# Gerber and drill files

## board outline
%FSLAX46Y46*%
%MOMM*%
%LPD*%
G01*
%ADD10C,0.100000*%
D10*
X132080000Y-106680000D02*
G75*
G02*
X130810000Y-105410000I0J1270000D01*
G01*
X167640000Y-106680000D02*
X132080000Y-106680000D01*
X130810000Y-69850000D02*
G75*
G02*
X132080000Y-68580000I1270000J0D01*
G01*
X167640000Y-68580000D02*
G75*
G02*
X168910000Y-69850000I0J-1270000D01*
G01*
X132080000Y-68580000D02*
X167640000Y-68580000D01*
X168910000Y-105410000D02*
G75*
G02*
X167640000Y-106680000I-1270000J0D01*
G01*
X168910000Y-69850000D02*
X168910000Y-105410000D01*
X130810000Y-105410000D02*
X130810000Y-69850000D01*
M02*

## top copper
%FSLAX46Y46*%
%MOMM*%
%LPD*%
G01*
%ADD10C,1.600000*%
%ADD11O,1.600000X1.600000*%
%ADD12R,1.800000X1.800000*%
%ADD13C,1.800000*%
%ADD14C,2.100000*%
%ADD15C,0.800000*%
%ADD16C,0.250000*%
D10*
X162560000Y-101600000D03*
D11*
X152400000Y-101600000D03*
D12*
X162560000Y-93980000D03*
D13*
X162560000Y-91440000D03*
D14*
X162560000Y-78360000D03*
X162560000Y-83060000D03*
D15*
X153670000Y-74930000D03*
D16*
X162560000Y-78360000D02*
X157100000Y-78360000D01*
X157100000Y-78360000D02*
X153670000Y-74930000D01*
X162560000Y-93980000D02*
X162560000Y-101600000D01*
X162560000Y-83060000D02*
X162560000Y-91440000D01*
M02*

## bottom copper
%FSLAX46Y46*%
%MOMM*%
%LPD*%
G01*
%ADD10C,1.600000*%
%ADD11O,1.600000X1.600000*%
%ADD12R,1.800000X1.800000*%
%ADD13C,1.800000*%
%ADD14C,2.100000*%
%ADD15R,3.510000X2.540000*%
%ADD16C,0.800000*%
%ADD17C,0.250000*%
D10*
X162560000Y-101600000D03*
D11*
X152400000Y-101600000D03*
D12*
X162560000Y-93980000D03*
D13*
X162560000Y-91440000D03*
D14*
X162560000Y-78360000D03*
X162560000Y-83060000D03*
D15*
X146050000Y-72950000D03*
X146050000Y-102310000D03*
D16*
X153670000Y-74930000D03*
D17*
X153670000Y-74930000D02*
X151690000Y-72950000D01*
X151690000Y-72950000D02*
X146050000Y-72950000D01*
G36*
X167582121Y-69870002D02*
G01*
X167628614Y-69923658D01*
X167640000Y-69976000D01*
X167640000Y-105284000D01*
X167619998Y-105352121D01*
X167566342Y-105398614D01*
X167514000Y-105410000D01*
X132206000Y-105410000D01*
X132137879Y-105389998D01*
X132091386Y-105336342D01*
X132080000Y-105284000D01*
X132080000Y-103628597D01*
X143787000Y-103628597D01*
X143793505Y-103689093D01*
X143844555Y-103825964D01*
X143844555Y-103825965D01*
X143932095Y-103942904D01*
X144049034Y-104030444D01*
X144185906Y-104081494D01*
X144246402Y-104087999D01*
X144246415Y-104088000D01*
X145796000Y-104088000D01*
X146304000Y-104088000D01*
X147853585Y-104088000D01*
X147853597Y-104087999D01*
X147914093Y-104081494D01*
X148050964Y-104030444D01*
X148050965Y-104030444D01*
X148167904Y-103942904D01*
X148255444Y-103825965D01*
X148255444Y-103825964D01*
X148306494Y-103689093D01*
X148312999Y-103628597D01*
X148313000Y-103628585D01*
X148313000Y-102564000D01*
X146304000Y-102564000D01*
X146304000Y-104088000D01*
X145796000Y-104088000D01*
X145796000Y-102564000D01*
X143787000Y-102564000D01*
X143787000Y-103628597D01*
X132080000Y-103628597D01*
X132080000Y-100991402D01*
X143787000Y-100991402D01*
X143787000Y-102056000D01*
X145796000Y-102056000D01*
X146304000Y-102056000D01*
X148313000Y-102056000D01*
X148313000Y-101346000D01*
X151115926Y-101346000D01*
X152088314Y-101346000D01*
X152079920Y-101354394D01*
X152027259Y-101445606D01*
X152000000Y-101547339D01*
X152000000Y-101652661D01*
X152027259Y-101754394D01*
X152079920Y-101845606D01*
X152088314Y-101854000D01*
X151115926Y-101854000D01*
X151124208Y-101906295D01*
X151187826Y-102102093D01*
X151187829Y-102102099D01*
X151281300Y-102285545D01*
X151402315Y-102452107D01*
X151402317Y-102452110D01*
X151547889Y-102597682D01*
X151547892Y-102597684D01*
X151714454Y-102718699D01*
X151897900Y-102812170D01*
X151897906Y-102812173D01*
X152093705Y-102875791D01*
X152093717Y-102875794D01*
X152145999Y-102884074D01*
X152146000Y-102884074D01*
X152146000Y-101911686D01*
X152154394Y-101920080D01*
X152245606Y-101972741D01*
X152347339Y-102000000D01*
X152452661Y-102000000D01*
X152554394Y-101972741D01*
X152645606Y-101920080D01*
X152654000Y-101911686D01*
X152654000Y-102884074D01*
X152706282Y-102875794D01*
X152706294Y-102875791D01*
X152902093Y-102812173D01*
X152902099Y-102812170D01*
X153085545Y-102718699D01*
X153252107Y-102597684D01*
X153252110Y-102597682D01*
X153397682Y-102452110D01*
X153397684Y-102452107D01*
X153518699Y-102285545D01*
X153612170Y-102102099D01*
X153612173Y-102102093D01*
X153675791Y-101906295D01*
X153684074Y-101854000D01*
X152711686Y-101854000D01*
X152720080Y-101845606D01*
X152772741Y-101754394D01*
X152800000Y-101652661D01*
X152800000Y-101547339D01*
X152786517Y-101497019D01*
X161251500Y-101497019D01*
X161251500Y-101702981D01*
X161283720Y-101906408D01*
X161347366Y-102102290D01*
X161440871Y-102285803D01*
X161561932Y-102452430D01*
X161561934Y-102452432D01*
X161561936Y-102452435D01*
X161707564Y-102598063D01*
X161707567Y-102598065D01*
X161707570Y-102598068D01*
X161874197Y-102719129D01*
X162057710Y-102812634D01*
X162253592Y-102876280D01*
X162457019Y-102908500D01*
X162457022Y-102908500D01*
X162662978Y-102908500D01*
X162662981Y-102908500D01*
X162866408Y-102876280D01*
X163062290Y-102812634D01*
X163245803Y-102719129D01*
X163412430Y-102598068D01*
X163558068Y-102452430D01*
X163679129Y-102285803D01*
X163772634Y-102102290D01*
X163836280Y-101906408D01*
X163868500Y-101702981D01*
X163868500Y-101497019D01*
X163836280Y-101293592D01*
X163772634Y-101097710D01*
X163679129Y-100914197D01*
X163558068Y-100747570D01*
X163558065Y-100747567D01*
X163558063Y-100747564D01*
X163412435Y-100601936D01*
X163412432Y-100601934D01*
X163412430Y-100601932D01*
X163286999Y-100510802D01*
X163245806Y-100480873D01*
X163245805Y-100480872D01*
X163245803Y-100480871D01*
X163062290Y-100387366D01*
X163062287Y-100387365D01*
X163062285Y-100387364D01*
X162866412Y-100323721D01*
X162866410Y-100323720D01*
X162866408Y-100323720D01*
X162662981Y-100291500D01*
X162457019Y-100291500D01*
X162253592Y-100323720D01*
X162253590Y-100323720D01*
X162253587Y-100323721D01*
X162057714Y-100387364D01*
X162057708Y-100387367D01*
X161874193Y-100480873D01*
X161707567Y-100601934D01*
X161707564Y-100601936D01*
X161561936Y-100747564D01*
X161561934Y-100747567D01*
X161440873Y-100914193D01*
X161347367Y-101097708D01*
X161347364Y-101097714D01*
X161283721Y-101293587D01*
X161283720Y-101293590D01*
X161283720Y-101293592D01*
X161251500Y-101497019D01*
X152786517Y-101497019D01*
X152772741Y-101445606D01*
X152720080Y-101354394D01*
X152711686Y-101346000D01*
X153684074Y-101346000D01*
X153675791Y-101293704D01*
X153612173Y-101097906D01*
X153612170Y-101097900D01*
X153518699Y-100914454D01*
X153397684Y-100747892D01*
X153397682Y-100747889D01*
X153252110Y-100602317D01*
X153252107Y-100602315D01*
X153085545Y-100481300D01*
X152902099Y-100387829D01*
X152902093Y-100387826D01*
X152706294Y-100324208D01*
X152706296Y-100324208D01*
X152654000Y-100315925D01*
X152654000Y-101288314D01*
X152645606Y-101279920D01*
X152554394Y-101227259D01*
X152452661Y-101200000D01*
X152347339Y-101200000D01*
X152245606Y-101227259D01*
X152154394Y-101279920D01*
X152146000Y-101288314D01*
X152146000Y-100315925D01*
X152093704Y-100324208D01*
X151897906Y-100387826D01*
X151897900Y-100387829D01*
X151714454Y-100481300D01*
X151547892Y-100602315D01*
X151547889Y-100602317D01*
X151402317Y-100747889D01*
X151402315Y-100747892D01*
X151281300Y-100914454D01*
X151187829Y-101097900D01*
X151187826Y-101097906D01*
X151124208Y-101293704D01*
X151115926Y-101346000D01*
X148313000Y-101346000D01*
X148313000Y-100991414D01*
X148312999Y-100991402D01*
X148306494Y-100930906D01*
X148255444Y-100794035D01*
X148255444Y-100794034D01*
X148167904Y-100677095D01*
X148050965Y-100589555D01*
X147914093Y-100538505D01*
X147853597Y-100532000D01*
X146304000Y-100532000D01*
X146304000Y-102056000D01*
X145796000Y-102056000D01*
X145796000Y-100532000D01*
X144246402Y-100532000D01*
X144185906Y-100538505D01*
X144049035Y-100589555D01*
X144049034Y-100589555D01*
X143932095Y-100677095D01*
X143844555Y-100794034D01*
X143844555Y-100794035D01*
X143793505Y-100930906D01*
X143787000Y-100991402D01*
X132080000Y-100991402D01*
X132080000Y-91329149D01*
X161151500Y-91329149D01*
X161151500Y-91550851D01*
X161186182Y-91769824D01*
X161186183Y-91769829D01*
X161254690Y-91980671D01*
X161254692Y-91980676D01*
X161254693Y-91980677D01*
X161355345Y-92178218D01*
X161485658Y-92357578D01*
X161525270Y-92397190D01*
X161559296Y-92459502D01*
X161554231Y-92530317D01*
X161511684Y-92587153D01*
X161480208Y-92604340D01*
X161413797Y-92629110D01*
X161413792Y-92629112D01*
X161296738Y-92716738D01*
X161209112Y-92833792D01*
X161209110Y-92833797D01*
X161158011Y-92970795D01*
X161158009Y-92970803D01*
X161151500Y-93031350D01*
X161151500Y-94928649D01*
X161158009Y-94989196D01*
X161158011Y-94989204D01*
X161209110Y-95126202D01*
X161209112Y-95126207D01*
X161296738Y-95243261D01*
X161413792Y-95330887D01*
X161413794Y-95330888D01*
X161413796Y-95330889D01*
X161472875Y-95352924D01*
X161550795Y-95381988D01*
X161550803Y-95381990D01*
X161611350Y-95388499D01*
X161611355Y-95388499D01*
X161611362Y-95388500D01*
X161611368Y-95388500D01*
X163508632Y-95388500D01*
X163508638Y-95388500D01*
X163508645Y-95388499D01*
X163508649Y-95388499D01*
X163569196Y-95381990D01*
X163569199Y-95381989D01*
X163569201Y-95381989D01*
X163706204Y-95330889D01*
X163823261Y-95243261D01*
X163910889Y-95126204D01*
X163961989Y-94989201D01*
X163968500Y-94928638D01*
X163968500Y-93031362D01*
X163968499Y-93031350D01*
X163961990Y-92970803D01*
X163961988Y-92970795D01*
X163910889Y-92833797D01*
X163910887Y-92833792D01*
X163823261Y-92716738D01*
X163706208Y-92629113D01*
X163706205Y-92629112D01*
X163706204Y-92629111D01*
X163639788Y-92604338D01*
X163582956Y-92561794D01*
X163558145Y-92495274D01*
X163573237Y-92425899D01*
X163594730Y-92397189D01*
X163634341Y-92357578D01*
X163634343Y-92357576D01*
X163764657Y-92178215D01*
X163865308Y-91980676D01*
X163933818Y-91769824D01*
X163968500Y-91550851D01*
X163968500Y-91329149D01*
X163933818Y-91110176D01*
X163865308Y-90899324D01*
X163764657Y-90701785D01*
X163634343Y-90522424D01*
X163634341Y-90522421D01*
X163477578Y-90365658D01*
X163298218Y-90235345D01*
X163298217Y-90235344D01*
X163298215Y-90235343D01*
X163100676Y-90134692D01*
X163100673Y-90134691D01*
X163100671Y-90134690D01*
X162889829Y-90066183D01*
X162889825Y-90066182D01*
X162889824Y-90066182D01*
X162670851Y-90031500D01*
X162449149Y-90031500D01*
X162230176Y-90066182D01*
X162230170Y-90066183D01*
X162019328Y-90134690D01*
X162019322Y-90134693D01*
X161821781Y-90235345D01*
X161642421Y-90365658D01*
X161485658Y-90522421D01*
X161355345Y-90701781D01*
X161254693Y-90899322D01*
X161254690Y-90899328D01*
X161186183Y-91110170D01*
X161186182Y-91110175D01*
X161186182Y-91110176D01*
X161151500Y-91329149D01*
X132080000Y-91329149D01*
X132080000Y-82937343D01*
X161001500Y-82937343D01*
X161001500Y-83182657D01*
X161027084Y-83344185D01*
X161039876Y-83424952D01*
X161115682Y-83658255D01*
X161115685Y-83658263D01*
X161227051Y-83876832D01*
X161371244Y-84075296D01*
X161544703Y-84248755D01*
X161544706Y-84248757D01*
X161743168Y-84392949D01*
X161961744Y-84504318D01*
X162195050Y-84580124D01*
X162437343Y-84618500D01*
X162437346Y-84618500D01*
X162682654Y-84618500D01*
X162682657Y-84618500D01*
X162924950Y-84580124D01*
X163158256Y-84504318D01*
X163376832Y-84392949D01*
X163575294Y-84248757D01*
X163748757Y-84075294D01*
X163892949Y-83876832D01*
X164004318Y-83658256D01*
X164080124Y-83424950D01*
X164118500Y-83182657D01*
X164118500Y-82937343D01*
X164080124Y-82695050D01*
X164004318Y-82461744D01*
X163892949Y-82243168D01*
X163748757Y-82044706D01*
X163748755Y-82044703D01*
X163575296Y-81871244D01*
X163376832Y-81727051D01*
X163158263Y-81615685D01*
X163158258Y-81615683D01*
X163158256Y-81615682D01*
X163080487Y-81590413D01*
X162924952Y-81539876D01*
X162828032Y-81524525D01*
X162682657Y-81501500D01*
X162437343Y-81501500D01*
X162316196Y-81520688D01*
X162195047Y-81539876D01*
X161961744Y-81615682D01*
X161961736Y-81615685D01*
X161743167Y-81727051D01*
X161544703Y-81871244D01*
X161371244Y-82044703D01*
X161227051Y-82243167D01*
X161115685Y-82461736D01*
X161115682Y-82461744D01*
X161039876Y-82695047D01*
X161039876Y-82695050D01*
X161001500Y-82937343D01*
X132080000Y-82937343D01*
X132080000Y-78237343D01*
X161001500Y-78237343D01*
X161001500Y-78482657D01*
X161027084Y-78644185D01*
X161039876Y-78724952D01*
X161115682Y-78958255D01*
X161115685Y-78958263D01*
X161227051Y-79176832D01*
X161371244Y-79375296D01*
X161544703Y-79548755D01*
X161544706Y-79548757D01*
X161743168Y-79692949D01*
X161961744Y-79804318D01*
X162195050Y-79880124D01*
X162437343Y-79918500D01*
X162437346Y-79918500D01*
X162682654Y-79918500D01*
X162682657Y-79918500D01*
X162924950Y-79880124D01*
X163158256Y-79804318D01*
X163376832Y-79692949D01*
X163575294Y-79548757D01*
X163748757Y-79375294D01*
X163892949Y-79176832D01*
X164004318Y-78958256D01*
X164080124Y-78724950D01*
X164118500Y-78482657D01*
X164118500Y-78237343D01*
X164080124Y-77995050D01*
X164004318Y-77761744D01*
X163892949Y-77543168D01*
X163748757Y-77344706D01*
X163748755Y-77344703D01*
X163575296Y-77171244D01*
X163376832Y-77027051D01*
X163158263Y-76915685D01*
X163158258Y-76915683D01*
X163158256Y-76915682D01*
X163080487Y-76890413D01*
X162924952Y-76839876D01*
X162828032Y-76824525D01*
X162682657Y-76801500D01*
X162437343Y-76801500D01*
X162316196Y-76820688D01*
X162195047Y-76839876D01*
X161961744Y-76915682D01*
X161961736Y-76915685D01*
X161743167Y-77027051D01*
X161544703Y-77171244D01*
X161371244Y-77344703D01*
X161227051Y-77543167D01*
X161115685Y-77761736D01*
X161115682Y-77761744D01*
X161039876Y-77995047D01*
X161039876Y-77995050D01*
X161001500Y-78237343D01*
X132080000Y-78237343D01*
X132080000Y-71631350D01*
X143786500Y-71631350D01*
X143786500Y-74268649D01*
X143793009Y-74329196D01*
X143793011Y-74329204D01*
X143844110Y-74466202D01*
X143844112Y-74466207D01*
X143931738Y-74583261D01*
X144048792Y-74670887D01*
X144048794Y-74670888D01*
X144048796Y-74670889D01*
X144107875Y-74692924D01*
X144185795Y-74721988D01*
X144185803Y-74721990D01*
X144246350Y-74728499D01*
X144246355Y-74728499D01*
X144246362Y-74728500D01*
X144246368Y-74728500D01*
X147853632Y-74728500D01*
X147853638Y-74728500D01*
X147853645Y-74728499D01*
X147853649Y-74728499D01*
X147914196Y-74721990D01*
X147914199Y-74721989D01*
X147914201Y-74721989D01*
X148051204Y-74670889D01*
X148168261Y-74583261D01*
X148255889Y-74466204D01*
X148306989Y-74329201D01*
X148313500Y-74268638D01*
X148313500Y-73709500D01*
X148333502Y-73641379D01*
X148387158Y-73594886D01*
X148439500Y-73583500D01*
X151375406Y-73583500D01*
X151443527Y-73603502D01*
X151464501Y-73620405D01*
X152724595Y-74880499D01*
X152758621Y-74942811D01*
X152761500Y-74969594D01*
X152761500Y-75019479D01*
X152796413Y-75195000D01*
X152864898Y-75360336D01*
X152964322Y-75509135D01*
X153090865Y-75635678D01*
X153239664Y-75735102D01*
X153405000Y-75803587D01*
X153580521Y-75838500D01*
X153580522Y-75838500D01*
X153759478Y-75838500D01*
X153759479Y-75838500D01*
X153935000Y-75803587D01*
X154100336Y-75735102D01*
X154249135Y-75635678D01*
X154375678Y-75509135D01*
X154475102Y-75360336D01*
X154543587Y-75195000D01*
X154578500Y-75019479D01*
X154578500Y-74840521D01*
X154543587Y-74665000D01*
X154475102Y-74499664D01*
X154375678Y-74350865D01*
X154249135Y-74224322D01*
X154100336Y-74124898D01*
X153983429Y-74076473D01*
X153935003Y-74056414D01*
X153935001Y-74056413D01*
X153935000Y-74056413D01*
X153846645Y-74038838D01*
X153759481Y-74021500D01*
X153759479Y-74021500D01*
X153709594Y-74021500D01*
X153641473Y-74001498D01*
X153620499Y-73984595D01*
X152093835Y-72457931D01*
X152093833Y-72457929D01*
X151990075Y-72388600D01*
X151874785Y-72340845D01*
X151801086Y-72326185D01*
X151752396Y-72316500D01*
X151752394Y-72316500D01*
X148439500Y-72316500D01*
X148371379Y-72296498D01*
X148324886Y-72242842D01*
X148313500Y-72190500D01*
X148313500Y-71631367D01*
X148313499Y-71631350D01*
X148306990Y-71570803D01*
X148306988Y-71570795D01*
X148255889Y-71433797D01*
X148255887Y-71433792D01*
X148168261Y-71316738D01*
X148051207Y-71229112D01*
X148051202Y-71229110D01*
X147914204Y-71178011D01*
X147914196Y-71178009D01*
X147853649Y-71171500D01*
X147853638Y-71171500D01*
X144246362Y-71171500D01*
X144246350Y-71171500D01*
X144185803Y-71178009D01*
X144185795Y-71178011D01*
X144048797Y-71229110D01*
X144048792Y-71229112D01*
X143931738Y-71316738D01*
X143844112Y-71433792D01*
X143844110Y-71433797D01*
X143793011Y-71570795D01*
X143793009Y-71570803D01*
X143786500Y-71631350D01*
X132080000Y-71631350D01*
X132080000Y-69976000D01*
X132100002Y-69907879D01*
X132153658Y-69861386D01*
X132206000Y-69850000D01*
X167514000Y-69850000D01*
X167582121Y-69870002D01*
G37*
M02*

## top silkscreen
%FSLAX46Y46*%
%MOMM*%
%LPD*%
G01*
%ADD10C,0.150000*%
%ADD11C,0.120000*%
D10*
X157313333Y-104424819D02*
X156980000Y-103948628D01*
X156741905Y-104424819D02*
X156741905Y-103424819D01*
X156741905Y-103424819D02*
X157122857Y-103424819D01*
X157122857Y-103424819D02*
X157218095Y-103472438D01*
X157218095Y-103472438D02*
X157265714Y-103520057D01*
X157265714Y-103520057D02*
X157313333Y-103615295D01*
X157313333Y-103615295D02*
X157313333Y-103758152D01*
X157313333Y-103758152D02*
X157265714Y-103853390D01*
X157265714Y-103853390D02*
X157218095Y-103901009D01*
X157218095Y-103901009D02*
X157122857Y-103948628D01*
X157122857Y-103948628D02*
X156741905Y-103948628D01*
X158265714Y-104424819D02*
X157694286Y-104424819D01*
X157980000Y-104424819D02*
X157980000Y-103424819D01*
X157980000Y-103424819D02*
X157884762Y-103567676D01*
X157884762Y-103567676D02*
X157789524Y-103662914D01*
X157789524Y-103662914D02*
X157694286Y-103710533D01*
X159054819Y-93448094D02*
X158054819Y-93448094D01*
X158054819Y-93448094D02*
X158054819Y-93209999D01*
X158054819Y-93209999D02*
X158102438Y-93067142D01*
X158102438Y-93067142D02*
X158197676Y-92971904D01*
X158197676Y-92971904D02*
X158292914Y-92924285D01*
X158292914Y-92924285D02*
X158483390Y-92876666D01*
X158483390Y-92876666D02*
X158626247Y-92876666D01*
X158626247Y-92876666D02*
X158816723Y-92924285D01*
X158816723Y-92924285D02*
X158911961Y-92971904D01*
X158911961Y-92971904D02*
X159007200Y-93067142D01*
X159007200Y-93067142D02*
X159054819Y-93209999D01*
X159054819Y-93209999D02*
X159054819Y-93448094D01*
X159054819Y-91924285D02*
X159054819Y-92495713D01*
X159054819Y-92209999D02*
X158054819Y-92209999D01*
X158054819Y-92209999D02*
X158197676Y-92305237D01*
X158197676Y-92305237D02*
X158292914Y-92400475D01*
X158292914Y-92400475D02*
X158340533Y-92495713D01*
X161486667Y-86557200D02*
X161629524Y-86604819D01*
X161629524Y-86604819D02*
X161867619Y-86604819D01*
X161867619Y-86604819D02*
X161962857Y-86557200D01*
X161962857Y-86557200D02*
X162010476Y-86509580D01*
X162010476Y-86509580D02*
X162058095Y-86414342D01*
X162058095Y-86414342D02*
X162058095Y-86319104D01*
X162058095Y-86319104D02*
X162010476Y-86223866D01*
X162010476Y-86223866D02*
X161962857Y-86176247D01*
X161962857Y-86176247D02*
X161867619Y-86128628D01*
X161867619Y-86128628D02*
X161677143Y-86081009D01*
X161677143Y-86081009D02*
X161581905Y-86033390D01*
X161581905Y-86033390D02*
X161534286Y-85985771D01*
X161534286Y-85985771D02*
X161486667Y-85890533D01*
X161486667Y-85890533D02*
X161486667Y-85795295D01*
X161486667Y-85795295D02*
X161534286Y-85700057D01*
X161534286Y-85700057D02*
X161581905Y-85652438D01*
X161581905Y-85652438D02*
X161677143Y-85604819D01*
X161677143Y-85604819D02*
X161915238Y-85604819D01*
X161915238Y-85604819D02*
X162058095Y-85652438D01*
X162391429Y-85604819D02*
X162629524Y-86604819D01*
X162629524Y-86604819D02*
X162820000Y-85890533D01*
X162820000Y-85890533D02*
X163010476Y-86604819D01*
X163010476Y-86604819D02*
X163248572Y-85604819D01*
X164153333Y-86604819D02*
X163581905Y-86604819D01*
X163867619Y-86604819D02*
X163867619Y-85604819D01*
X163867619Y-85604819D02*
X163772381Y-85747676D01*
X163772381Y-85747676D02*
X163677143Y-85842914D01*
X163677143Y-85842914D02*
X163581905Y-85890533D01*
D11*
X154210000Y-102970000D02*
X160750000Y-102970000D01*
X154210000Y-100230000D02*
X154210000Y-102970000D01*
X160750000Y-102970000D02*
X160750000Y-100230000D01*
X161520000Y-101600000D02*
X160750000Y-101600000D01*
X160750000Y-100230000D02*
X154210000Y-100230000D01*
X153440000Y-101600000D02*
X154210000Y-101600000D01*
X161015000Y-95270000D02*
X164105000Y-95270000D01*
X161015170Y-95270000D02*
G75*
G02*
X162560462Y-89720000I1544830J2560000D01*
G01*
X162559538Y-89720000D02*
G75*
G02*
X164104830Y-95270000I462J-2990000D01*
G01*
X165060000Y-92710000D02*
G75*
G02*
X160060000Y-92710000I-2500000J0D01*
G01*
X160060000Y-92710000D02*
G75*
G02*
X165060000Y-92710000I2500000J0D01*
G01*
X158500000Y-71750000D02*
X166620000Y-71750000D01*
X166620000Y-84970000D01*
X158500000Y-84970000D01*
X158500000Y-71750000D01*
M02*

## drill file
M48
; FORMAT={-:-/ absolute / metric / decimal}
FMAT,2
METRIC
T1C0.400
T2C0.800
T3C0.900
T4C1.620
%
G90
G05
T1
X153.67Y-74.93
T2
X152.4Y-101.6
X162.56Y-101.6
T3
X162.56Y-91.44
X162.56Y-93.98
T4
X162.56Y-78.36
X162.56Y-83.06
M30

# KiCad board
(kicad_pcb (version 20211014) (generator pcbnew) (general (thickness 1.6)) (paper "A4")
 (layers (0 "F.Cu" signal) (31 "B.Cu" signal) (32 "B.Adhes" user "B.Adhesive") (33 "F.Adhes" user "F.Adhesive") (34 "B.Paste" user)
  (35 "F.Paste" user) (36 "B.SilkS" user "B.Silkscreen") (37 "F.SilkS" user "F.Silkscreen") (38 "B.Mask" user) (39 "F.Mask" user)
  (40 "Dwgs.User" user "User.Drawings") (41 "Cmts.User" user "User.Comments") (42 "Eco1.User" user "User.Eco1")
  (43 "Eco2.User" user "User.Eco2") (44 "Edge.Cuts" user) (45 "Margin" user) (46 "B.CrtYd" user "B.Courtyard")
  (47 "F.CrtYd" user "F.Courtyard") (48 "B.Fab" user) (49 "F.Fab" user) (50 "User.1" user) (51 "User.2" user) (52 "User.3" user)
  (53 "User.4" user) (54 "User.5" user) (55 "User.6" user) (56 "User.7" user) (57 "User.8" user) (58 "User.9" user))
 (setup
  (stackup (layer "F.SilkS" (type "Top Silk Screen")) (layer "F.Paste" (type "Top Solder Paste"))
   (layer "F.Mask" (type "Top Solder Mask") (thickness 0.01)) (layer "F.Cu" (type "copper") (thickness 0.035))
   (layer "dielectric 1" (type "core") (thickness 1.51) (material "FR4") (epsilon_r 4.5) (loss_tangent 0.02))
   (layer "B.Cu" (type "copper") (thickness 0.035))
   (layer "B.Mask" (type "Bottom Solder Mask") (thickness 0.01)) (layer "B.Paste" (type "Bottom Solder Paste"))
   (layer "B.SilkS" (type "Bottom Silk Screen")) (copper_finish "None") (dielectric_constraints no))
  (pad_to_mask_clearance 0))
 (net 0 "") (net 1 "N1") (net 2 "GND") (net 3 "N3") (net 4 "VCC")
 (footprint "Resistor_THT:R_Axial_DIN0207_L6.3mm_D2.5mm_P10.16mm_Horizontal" (layer "F.Cu") (at 162.56 101.6 180)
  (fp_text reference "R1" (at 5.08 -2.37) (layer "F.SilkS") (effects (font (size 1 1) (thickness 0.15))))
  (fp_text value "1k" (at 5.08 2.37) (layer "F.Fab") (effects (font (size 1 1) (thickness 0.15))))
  (fp_line (start 8.35 -1.37) (end 1.81 -1.37) (layer "F.SilkS") (width 0.12))
  (fp_line (start 8.35 1.37) (end 8.35 -1.37) (layer "F.SilkS") (width 0.12))
  (fp_line (start 1.81 -1.37) (end 1.81 1.37) (layer "F.SilkS") (width 0.12))
  (fp_line (start 1.04 0) (end 1.81 0) (layer "F.SilkS") (width 0.12))
  (fp_line (start 1.81 1.37) (end 8.35 1.37) (layer "F.SilkS") (width 0.12))
  (fp_line (start 9.12 0) (end 8.35 0) (layer "F.SilkS") (width 0.12))
  (pad "1" thru_hole circle (at 0 0 180) (size 1.6 1.6) (drill 0.8) (layers *.Cu *.Mask) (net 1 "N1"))
  (pad "2" thru_hole oval (at 10.16 0 180) (size 1.6 1.6) (drill 0.8) (layers *.Cu *.Mask) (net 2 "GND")))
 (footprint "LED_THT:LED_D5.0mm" (layer "F.Cu") (at 162.56 93.98 90)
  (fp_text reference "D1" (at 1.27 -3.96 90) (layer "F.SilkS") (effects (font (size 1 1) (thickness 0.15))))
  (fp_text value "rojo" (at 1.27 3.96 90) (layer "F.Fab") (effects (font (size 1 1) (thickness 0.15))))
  (fp_line (start -1.29 -1.545) (end -1.29 1.545) (layer "F.SilkS") (width 0.12))
  (fp_arc (start -1.29 -1.54483) (mid 2.072002 -2.880433) (end 4.26 0.000462) (layer "F.SilkS") (width 0.12))
  (fp_arc (start 4.26 -0.000462) (mid 2.072002 2.880433) (end -1.29 1.54483) (layer "F.SilkS") (width 0.12))
  (fp_circle (center 1.27 0) (end 3.77 0) (layer "F.SilkS") (width 0.12) (fill none))
  (pad "1" thru_hole rect (at 0 0 90) (size 1.8 1.8) (drill 0.9) (layers *.Cu *.Mask) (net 1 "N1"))
  (pad "2" thru_hole circle (at 2.54 0 90) (size 1.8 1.8) (drill 0.9) (layers *.Cu *.Mask) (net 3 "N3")))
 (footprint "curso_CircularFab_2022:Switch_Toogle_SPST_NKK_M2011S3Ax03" (layer "F.Cu") (at 162.56 73.66)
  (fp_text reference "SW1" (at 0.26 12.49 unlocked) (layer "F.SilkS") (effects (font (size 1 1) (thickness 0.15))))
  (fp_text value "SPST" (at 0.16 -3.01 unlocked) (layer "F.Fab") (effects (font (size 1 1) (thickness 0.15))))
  (fp_rect (start -4.06 -1.91) (end 4.06 11.31) (layer "F.SilkS") (width 0.12) (fill none))
  (pad "2" thru_hole circle (at 0 4.7) (size 2.1 2.1) (drill 1.62) (layers *.Cu *.Mask) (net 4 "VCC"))
  (pad "3" thru_hole circle (at 0 9.4) (size 2.1 2.1) (drill 1.62) (layers *.Cu *.Mask) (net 3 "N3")))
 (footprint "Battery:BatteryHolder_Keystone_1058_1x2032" (layer "B.Cu") (at 146.05 87.63 -90)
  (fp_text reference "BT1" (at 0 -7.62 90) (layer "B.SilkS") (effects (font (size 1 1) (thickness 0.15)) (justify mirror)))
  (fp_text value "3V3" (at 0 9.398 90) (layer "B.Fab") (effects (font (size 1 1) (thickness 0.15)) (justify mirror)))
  (pad "1" smd rect (at -14.68 0 270) (size 2.54 3.51) (layers "B.Cu" "B.Paste" "B.Mask") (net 4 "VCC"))
  (pad "2" smd rect (at 14.68 0 270) (size 2.54 3.51) (layers "B.Cu" "B.Paste" "B.Mask") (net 2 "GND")))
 (gr_arc (start 132.08 106.68) (mid 131.181974 106.308026) (end 130.81 105.41) (layer "Edge.Cuts") (width 0.1))
 (gr_line (start 167.64 106.68) (end 132.08 106.68) (layer "Edge.Cuts") (width 0.1))
 (gr_arc (start 130.81 69.85) (mid 131.181974 68.951974) (end 132.08 68.58) (layer "Edge.Cuts") (width 0.1))
 (gr_arc (start 167.64 68.58) (mid 168.538026 68.951974) (end 168.91 69.85) (layer "Edge.Cuts") (width 0.1))
 (gr_line (start 132.08 68.58) (end 167.64 68.58) (layer "Edge.Cuts") (width 0.1))
 (gr_arc (start 168.91 105.41) (mid 168.538026 106.308026) (end 167.64 106.68) (layer "Edge.Cuts") (width 0.1))
 (gr_line (start 168.91 69.85) (end 168.91 105.41) (layer "Edge.Cuts") (width 0.1))
 (gr_line (start 130.81 105.41) (end 130.81 69.85) (layer "Edge.Cuts") (width 0.1))
 (segment (start 162.56 78.36) (end 157.1 78.36) (width 0.25) (layer "F.Cu") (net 4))
 (segment (start 157.1 78.36) (end 153.67 74.93) (width 0.25) (layer "F.Cu") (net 4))
 (via (at 153.67 74.93) (size 0.8) (drill 0.4) (layers "F.Cu" "B.Cu") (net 4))
 (segment (start 153.67 74.93) (end 151.69 72.95) (width 0.25) (layer "B.Cu") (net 4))
 (segment (start 151.69 72.95) (end 146.05 72.95) (width 0.25) (layer "B.Cu") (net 4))
 (segment (start 162.56 93.98) (end 162.56 101.6) (width 0.25) (layer "F.Cu") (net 1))
 (segment (start 162.56 83.06) (end 162.56 91.44) (width 0.25) (layer "F.Cu") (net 3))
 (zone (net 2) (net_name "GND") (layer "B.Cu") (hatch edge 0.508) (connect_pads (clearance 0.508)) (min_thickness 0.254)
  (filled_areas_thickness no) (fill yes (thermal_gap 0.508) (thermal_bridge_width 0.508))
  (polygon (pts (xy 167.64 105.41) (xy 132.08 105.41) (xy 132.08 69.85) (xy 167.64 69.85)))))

